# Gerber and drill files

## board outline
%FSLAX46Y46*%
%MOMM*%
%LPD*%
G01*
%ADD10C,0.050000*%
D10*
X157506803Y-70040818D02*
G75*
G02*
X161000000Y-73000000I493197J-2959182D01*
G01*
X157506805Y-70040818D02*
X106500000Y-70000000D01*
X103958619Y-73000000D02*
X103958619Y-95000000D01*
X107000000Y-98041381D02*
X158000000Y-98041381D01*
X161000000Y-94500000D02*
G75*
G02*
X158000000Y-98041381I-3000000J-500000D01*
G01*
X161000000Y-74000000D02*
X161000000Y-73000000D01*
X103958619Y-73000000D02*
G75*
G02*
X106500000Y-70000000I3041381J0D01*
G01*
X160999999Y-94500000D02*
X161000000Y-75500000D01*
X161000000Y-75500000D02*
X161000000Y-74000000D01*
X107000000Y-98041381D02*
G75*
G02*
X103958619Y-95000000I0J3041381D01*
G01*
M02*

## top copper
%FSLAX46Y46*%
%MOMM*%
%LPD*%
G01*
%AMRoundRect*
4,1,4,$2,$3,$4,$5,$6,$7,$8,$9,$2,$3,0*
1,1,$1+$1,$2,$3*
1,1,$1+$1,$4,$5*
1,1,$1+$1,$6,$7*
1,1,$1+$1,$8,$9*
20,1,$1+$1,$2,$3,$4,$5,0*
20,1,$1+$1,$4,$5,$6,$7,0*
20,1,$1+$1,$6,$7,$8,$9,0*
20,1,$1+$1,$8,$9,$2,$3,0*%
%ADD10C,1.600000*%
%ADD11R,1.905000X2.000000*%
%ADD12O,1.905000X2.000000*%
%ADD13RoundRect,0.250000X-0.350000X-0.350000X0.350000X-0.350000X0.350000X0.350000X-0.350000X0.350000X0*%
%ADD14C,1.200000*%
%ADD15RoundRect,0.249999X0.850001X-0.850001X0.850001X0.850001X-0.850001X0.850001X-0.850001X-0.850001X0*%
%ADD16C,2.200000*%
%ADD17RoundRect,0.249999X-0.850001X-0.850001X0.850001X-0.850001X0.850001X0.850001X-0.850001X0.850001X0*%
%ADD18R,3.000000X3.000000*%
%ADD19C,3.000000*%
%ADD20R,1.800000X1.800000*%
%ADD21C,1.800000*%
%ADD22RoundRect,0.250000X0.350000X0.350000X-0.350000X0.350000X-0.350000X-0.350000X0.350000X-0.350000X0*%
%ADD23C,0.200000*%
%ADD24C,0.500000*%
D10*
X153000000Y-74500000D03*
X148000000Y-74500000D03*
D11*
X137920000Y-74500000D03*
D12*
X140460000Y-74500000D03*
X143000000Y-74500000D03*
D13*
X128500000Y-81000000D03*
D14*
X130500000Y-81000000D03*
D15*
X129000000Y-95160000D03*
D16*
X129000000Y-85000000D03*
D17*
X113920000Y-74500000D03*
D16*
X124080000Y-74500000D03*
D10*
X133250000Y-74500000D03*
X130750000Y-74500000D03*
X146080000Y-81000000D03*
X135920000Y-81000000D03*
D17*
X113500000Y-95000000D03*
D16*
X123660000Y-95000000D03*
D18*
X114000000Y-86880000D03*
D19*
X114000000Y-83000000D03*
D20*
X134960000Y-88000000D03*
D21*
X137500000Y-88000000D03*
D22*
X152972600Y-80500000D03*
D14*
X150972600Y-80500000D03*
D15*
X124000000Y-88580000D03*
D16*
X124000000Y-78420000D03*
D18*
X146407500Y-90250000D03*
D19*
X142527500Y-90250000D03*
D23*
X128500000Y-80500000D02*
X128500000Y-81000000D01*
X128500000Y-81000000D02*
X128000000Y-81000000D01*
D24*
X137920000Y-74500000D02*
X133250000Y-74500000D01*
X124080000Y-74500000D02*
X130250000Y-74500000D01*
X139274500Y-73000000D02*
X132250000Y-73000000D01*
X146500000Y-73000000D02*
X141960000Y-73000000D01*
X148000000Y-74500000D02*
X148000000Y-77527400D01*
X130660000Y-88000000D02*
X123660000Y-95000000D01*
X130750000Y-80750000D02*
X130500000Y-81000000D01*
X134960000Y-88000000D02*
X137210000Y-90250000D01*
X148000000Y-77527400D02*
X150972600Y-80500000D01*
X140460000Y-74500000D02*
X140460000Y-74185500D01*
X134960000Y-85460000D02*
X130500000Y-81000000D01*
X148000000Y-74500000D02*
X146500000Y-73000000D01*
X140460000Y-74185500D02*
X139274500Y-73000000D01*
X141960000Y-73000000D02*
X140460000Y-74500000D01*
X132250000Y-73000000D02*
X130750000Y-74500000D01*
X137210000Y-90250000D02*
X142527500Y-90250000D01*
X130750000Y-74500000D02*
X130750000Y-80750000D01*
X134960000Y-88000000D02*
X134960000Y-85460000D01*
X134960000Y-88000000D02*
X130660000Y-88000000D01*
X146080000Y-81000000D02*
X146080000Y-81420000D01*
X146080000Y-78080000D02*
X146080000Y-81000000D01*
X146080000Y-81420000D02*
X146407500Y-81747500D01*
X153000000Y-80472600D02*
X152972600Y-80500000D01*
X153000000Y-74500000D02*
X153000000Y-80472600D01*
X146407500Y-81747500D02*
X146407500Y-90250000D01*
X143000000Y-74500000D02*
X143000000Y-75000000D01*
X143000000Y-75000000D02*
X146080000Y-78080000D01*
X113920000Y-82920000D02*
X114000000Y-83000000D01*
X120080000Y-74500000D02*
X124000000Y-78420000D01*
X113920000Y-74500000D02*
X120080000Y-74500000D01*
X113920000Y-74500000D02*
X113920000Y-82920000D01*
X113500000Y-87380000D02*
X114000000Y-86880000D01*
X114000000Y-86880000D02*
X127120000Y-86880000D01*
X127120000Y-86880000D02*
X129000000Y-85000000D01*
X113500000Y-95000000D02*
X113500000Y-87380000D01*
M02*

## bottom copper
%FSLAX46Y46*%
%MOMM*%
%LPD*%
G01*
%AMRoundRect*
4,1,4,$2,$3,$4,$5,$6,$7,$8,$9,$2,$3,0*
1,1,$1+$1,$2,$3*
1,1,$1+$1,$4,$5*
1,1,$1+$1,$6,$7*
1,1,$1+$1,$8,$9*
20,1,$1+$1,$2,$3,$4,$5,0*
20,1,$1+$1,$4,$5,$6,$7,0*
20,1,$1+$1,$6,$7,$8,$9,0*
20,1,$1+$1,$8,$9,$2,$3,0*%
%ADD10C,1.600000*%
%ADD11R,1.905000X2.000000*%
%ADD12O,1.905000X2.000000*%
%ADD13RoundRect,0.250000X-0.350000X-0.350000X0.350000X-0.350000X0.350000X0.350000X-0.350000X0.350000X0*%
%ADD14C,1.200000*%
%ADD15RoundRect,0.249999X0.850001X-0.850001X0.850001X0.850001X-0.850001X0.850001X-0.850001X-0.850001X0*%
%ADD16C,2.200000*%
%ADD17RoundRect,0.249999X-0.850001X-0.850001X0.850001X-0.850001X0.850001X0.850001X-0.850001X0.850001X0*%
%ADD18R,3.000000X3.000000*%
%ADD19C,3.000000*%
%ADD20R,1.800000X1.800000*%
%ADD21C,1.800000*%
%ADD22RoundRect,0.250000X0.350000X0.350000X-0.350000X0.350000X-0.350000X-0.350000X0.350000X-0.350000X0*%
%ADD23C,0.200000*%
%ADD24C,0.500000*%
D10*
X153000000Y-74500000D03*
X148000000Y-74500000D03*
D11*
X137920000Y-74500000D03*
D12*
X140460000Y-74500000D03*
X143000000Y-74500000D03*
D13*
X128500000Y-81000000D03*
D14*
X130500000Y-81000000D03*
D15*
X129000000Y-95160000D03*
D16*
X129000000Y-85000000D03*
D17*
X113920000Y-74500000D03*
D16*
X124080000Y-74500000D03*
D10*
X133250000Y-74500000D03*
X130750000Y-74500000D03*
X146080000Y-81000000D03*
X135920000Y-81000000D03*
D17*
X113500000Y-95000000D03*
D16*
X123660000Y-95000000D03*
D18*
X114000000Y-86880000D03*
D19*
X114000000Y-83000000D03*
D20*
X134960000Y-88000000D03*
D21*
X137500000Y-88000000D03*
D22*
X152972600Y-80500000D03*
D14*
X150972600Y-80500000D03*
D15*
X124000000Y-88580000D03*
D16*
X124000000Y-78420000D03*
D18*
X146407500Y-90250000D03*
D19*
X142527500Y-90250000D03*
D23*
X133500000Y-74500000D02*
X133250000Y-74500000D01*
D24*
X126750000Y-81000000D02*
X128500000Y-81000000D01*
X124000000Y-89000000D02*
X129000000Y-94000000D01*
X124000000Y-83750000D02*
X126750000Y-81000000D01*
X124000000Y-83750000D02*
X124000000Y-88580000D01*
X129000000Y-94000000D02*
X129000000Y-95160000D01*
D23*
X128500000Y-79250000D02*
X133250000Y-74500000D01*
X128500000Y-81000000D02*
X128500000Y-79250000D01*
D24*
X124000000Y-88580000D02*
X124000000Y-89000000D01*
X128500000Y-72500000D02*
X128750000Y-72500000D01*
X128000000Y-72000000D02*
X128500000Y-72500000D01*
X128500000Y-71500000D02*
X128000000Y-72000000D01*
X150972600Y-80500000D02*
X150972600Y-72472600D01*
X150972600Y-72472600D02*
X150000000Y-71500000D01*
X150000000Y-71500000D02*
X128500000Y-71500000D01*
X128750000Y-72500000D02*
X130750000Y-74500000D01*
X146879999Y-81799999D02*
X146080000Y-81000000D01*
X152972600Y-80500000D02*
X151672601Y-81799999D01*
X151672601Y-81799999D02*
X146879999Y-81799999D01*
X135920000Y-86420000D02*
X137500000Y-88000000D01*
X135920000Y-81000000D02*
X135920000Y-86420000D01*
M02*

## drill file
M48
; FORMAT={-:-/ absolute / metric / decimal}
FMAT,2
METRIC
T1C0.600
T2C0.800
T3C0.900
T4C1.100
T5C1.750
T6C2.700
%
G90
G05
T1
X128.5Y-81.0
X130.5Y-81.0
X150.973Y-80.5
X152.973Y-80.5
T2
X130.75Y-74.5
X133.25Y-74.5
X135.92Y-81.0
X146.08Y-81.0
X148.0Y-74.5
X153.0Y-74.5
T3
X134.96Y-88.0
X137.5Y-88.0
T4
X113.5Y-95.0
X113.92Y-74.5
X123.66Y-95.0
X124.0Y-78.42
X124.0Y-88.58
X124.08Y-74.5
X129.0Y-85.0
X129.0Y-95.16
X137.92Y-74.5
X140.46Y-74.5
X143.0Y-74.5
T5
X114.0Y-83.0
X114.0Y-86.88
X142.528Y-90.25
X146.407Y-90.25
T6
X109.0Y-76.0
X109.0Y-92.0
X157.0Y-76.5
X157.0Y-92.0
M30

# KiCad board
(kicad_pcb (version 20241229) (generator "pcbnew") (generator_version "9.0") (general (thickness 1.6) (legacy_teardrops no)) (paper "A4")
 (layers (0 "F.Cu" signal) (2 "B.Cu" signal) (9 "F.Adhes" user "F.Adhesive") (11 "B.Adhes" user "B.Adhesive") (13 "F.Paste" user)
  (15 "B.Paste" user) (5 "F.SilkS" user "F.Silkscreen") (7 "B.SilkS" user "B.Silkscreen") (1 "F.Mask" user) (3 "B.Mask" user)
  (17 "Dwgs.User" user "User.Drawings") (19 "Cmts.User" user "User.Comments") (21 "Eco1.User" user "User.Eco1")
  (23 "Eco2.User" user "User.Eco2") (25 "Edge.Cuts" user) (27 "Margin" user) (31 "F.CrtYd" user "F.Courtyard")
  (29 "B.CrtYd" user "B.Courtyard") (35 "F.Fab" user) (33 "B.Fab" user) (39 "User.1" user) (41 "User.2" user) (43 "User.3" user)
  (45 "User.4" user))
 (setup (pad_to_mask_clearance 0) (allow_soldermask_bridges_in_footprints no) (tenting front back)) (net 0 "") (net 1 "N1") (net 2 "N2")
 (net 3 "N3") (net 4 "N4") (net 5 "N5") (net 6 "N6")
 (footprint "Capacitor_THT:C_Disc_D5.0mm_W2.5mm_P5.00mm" (layer "F.Cu") (at 153 74.5 180)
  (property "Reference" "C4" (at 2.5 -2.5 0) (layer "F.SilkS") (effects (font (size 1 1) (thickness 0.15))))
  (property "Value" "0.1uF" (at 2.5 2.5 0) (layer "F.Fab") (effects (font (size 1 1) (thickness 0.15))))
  (pad "1" thru_hole circle (at 0 0 180) (size 1.6 1.6) (drill 0.8) (layers "*.Cu" "*.Mask") (remove_unused_layers no) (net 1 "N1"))
  (pad "2" thru_hole circle (at 5 0 180) (size 1.6 1.6) (drill 0.8) (layers "*.Cu" "*.Mask") (remove_unused_layers no) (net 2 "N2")))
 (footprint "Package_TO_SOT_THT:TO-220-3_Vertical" (layer "F.Cu") (at 137.92 74.5)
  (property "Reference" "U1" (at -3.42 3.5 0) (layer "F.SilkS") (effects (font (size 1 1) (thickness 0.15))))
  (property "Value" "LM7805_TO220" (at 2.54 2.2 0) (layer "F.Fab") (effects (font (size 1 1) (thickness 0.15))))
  (pad "1" thru_hole rect (at 0 0) (size 1.905 2) (drill 1.1) (layers "*.Cu" "*.Mask") (remove_unused_layers no) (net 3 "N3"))
  (pad "2" thru_hole oval (at 2.54 0) (size 1.905 2) (drill 1.1) (layers "*.Cu" "*.Mask") (remove_unused_layers no) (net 2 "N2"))
  (pad "3" thru_hole oval (at 5.08 0) (size 1.905 2) (drill 1.1) (layers "*.Cu" "*.Mask") (remove_unused_layers no) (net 1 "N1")))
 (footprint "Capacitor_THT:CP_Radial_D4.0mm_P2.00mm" (layer "F.Cu") (at 128.5 81)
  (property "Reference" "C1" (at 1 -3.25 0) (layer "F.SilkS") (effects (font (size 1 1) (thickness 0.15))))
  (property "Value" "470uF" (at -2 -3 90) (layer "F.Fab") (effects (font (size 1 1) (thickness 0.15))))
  (pad "1" thru_hole roundrect (at 0 0) (size 1.2 1.2) (drill 0.6) (layers "*.Cu" "*.Mask") (remove_unused_layers no)
   (roundrect_rratio 0.208333) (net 3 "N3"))
  (pad "2" thru_hole circle (at 2 0) (size 1.2 1.2) (drill 0.6) (layers "*.Cu" "*.Mask") (remove_unused_layers no) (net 2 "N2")))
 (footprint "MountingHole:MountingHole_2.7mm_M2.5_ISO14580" (layer "F.Cu") (at 109 76)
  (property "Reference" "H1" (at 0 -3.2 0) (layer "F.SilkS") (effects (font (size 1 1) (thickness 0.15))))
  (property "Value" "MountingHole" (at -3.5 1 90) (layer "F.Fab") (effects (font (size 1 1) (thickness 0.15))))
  (pad "" np_thru_hole circle (at 0 0) (size 2.7 2.7) (drill 2.7) (layers "*.Cu" "*.Mask")))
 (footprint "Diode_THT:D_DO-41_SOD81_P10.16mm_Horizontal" (layer "F.Cu") (at 129 95.16 90)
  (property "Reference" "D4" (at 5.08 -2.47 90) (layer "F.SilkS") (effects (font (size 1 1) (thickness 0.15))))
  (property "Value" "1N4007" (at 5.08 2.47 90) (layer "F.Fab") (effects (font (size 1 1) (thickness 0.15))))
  (pad "1" thru_hole roundrect (at 0 0 90) (size 2.2 2.2) (drill 1.1) (layers "*.Cu" "*.Mask") (remove_unused_layers no)
   (roundrect_rratio 0.113636) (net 3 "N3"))
  (pad "2" thru_hole circle (at 10.16 0 90) (size 2.2 2.2) (drill 1.1) (layers "*.Cu" "*.Mask") (remove_unused_layers no) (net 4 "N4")))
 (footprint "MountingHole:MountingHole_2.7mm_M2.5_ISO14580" (layer "F.Cu") (at 109 92 180)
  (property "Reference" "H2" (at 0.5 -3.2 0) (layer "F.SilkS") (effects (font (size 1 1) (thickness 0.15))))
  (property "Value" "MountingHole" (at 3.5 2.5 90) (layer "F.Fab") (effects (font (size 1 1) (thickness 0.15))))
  (pad "" np_thru_hole circle (at 0 0 180) (size 2.7 2.7) (drill 2.7) (layers "*.Cu" "*.Mask")))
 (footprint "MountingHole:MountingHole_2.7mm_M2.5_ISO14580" (layer "F.Cu") (at 157 92 90)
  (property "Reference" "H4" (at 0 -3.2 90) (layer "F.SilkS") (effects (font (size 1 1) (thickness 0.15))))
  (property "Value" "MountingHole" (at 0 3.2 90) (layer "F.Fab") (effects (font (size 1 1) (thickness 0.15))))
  (pad "" np_thru_hole circle (at 0 0 90) (size 2.7 2.7) (drill 2.7) (layers "*.Cu" "*.Mask")))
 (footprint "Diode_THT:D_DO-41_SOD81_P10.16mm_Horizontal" (layer "F.Cu") (at 113.92 74.5)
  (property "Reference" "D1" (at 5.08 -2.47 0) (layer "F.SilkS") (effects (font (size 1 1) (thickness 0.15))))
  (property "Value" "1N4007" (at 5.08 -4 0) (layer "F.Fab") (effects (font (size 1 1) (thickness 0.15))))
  (pad "1" thru_hole roundrect (at 0 0) (size 2.2 2.2) (drill 1.1) (layers "*.Cu" "*.Mask") (remove_unused_layers no)
   (roundrect_rratio 0.113636) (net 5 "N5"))
  (pad "2" thru_hole circle (at 10.16 0) (size 2.2 2.2) (drill 1.1) (layers "*.Cu" "*.Mask") (remove_unused_layers no) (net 2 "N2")))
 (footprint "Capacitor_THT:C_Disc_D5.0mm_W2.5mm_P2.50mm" (layer "F.Cu") (at 133.25 74.5 180)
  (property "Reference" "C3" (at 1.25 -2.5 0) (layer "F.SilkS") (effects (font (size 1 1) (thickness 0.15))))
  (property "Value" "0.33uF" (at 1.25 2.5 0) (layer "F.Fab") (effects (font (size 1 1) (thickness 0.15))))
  (pad "1" thru_hole circle (at 0 0 180) (size 1.6 1.6) (drill 0.8) (layers "*.Cu" "*.Mask") (remove_unused_layers no) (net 3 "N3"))
  (pad "2" thru_hole circle (at 2.5 0 180) (size 1.6 1.6) (drill 0.8) (layers "*.Cu" "*.Mask") (remove_unused_layers no) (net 2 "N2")))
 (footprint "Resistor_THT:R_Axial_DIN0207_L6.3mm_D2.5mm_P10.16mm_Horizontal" (layer "F.Cu") (at 146.08 81 180)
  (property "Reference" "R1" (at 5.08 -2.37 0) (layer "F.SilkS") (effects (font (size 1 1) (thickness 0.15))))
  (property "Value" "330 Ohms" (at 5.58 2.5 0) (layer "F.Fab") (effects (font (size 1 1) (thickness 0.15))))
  (pad "1" thru_hole circle (at 0 0 180) (size 1.6 1.6) (drill 0.8) (layers "*.Cu" "*.Mask") (remove_unused_layers no) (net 1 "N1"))
  (pad "2" thru_hole circle (at 10.16 0 180) (size 1.6 1.6) (drill 0.8) (layers "*.Cu" "*.Mask") (remove_unused_layers no) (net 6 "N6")))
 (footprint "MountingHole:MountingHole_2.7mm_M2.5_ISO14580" (layer "F.Cu") (at 157 76.5 90)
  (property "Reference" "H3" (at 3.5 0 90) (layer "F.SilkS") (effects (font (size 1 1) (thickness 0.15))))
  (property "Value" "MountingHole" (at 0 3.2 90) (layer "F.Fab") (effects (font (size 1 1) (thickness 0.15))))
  (pad "" np_thru_hole circle (at 0 0 90) (size 2.7 2.7) (drill 2.7) (layers "*.Cu" "*.Mask")))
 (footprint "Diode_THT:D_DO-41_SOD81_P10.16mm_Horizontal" (layer "F.Cu") (at 113.5 95)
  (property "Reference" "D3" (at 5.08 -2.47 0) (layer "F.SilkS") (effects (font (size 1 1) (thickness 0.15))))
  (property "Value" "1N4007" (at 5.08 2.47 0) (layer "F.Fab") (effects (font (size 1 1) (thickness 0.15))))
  (pad "1" thru_hole roundrect (at 0 0) (size 2.2 2.2) (drill 1.1) (layers "*.Cu" "*.Mask") (remove_unused_layers no)
   (roundrect_rratio 0.113636) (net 4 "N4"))
  (pad "2" thru_hole circle (at 10.16 0) (size 2.2 2.2) (drill 1.1) (layers "*.Cu" "*.Mask") (remove_unused_layers no) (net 2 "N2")))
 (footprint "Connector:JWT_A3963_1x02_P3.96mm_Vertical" (layer "F.Cu") (at 114 86.88 90)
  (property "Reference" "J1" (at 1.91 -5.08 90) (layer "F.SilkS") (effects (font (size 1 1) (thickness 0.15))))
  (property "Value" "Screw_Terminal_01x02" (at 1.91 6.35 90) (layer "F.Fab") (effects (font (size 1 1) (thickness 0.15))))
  (pad "1" thru_hole rect (at 0 0 90) (size 3 3) (drill 1.75) (layers "*.Cu" "*.Mask") (remove_unused_layers no) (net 4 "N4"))
  (pad "2" thru_hole circle (at 3.88 0 90) (size 3 3) (drill 1.75) (layers "*.Cu" "*.Mask") (remove_unused_layers no) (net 5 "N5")))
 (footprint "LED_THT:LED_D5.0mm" (layer "F.Cu") (at 134.96 88)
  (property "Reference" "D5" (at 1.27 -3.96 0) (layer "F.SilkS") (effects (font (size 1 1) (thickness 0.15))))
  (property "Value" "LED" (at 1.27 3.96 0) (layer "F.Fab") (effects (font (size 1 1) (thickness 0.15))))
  (pad "1" thru_hole rect (at 0 0) (size 1.8 1.8) (drill 0.9) (layers "*.Cu" "*.Mask") (remove_unused_layers no) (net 2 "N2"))
  (pad "2" thru_hole circle (at 2.54 0) (size 1.8 1.8) (drill 0.9) (layers "*.Cu" "*.Mask") (remove_unused_layers no) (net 6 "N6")))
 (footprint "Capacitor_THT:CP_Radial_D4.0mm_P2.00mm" (layer "F.Cu") (at 152.9726 80.5 180)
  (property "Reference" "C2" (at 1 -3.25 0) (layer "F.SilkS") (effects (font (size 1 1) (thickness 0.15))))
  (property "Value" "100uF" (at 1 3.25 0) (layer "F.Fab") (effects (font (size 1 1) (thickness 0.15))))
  (pad "1" thru_hole roundrect (at 0 0 180) (size 1.2 1.2) (drill 0.6) (layers "*.Cu" "*.Mask") (remove_unused_layers no)
   (roundrect_rratio 0.208333) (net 1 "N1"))
  (pad "2" thru_hole circle (at 2 0 180) (size 1.2 1.2) (drill 0.6) (layers "*.Cu" "*.Mask") (remove_unused_layers no) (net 2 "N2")))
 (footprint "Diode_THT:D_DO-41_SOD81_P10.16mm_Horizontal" (layer "F.Cu") (at 124 88.58 90)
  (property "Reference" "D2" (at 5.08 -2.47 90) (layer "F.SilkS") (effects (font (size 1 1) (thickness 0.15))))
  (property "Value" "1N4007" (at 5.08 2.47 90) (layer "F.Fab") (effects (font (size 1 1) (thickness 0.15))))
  (pad "1" thru_hole roundrect (at 0 0 90) (size 2.2 2.2) (drill 1.1) (layers "*.Cu" "*.Mask") (remove_unused_layers no)
   (roundrect_rratio 0.113636) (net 3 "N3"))
  (pad "2" thru_hole circle (at 10.16 0 90) (size 2.2 2.2) (drill 1.1) (layers "*.Cu" "*.Mask") (remove_unused_layers no) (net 5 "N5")))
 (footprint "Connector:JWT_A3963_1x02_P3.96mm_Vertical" (layer "F.Cu") (at 146.4075 90.25 180)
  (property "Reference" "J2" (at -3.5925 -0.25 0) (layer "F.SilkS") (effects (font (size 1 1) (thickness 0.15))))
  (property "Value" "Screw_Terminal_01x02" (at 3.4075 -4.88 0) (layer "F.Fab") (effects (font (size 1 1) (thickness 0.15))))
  (pad "1" thru_hole rect (at 0 0 180) (size 3 3) (drill 1.75) (layers "*.Cu" "*.Mask") (remove_unused_layers no) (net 1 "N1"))
  (pad "2" thru_hole circle (at 3.88 0 180) (size 3 3) (drill 1.75) (layers "*.Cu" "*.Mask") (remove_unused_layers no) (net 2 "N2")))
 (gr_arc (start 157.506803 70.040818) (mid 159.939125 70.71094) (end 161 73) (stroke (width 0.05) (type default)) (layer "Edge.Cuts"))
 (gr_line (start 157.506805 70.040818) (end 106.5 70) (stroke (width 0.05) (type default)) (layer "Edge.Cuts"))
 (gr_line (start 103.958619 73) (end 103.958619 95) (stroke (width 0.05) (type default)) (layer "Edge.Cuts"))
 (gr_line (start 107 98.041381) (end 158 98.041381) (stroke (width 0.05) (type default)) (layer "Edge.Cuts"))
 (gr_arc (start 161 94.5) (mid 160.320635 96.965872) (end 158 98.041381) (stroke (width 0.05) (type default)) (layer "Edge.Cuts"))
 (gr_line (start 161 74) (end 161 73) (stroke (width 0.05) (type default)) (layer "Edge.Cuts"))
 (gr_arc (start 103.958619 73) (mid 104.679366 71.034128) (end 106.5 70) (stroke (width 0.05) (type default)) (layer "Edge.Cuts"))
 (gr_line (start 160.999999 94.5) (end 161 75.5) (stroke (width 0.05) (type default)) (layer "Edge.Cuts"))
 (gr_line (start 161 75.5) (end 161 74) (stroke (width 0.05) (type default)) (layer "Edge.Cuts"))
 (gr_arc (start 107 98.041381) (mid 104.849419 97.150581) (end 103.958619 95) (stroke (width 0.05) (type default)) (layer "Edge.Cuts"))
 (segment (start 128.5 80.5) (end 128.5 81) (width 0.2) (layer "F.Cu") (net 3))
 (segment (start 128.5 81) (end 128 81) (width 0.2) (layer "F.Cu") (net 3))
 (segment (start 137.92 74.5) (end 133.25 74.5) (width 0.5) (layer "F.Cu") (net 3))
 (segment (start 133.5 74.5) (end 133.25 74.5) (width 0.2) (layer "B.Cu") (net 3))
 (segment (start 126.75 81) (end 128.5 81) (width 0.5) (layer "B.Cu") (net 3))
 (segment (start 124 89) (end 129 94) (width 0.5) (layer "B.Cu") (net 3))
 (segment (start 124 83.75) (end 126.75 81) (width 0.5) (layer "B.Cu") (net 3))
 (segment (start 124 83.75) (end 124 88.58) (width 0.5) (layer "B.Cu") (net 3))
 (segment (start 129 94) (end 129 95.16) (width 0.5) (layer "B.Cu") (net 3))
 (segment (start 128.5 79.25) (end 133.25 74.5) (width 0.2) (layer "B.Cu") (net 3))
 (segment (start 128.5 81) (end 128.5 79.25) (width 0.2) (layer "B.Cu") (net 3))
 (segment (start 124 88.58) (end 124 89) (width 0.5) (layer "B.Cu") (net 3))
 (segment (start 124.08 74.5) (end 130.25 74.5) (width 0.5) (layer "F.Cu") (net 2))
 (segment (start 139.2745 73) (end 132.25 73) (width 0.5) (layer "F.Cu") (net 2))
 (segment (start 146.5 73) (end 141.96 73) (width 0.5) (layer "F.Cu") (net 2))
 (segment (start 148 74.5) (end 148 77.5274) (width 0.5) (layer "F.Cu") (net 2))
 (segment (start 130.66 88) (end 123.66 95) (width 0.5) (layer "F.Cu") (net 2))
 (segment (start 130.75 80.75) (end 130.5 81) (width 0.5) (layer "F.Cu") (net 2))
 (segment (start 134.96 88) (end 137.21 90.25) (width 0.5) (layer "F.Cu") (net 2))
 (segment (start 148 77.5274) (end 150.9726 80.5) (width 0.5) (layer "F.Cu") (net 2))
 (segment (start 140.46 74.5) (end 140.46 74.1855) (width 0.5) (layer "F.Cu") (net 2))
 (segment (start 134.96 85.46) (end 130.5 81) (width 0.5) (layer "F.Cu") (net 2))
 (segment (start 148 74.5) (end 146.5 73) (width 0.5) (layer "F.Cu") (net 2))
 (segment (start 140.46 74.1855) (end 139.2745 73) (width 0.5) (layer "F.Cu") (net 2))
 (segment (start 141.96 73) (end 140.46 74.5) (width 0.5) (layer "F.Cu") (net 2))
 (segment (start 132.25 73) (end 130.75 74.5) (width 0.5) (layer "F.Cu") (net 2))
 (segment (start 137.21 90.25) (end 142.5275 90.25) (width 0.5) (layer "F.Cu") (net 2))
 (segment (start 130.75 74.5) (end 130.75 80.75) (width 0.5) (layer "F.Cu") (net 2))
 (segment (start 134.96 88) (end 134.96 85.46) (width 0.5) (layer "F.Cu") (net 2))
 (segment (start 134.96 88) (end 130.66 88) (width 0.5) (layer "F.Cu") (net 2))
 (segment (start 128.5 72.5) (end 128.75 72.5) (width 0.5) (layer "B.Cu") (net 2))
 (segment (start 128 72) (end 128.5 72.5) (width 0.5) (layer "B.Cu") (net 2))
 (segment (start 128.5 71.5) (end 128 72) (width 0.5) (layer "B.Cu") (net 2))
 (segment (start 150.9726 80.5) (end 150.9726 72.4726) (width 0.5) (layer "B.Cu") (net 2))
 (segment (start 150.9726 72.4726) (end 150 71.5) (width 0.5) (layer "B.Cu") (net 2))
 (segment (start 150 71.5) (end 128.5 71.5) (width 0.5) (layer "B.Cu") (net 2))
 (segment (start 128.75 72.5) (end 130.75 74.5) (width 0.5) (layer "B.Cu") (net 2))
 (segment (start 146.08 81) (end 146.08 81.42) (width 0.5) (layer "F.Cu") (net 1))
 (segment (start 146.08 78.08) (end 146.08 81) (width 0.5) (layer "F.Cu") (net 1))
 (segment (start 146.08 81.42) (end 146.4075 81.7475) (width 0.5) (layer "F.Cu") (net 1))
 (segment (start 153 80.4726) (end 152.9726 80.5) (width 0.5) (layer "F.Cu") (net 1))
 (segment (start 153 74.5) (end 153 80.4726) (width 0.5) (layer "F.Cu") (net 1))
 (segment (start 146.4075 81.7475) (end 146.4075 90.25) (width 0.5) (layer "F.Cu") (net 1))
 (segment (start 143 74.5) (end 143 75) (width 0.5) (layer "F.Cu") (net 1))
 (segment (start 143 75) (end 146.08 78.08) (width 0.5) (layer "F.Cu") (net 1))
 (segment (start 146.879999 81.799999) (end 146.08 81) (width 0.5) (layer "B.Cu") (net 1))
 (segment (start 152.9726 80.5) (end 151.672601 81.799999) (width 0.5) (layer "B.Cu") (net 1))
 (segment (start 151.672601 81.799999) (end 146.879999 81.799999) (width 0.5) (layer "B.Cu") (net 1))
 (segment (start 113.92 82.92) (end 114 83) (width 0.5) (layer "F.Cu") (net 5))
 (segment (start 120.08 74.5) (end 124 78.42) (width 0.5) (layer "F.Cu") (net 5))
 (segment (start 113.92 74.5) (end 120.08 74.5) (width 0.5) (layer "F.Cu") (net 5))
 (segment (start 113.92 74.5) (end 113.92 82.92) (width 0.5) (layer "F.Cu") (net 5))
 (segment (start 113.5 87.38) (end 114 86.88) (width 0.5) (layer "F.Cu") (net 4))
 (segment (start 114 86.88) (end 127.12 86.88) (width 0.5) (layer "F.Cu") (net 4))
 (segment (start 127.12 86.88) (end 129 85) (width 0.5) (layer "F.Cu") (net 4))
 (segment (start 113.5 95) (end 113.5 87.38) (width 0.5) (layer "F.Cu") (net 4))
 (segment (start 135.92 86.42) (end 137.5 88) (width 0.5) (layer "B.Cu") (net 6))
 (segment (start 135.92 81) (end 135.92 86.42) (width 0.5) (layer "B.Cu") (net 6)))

